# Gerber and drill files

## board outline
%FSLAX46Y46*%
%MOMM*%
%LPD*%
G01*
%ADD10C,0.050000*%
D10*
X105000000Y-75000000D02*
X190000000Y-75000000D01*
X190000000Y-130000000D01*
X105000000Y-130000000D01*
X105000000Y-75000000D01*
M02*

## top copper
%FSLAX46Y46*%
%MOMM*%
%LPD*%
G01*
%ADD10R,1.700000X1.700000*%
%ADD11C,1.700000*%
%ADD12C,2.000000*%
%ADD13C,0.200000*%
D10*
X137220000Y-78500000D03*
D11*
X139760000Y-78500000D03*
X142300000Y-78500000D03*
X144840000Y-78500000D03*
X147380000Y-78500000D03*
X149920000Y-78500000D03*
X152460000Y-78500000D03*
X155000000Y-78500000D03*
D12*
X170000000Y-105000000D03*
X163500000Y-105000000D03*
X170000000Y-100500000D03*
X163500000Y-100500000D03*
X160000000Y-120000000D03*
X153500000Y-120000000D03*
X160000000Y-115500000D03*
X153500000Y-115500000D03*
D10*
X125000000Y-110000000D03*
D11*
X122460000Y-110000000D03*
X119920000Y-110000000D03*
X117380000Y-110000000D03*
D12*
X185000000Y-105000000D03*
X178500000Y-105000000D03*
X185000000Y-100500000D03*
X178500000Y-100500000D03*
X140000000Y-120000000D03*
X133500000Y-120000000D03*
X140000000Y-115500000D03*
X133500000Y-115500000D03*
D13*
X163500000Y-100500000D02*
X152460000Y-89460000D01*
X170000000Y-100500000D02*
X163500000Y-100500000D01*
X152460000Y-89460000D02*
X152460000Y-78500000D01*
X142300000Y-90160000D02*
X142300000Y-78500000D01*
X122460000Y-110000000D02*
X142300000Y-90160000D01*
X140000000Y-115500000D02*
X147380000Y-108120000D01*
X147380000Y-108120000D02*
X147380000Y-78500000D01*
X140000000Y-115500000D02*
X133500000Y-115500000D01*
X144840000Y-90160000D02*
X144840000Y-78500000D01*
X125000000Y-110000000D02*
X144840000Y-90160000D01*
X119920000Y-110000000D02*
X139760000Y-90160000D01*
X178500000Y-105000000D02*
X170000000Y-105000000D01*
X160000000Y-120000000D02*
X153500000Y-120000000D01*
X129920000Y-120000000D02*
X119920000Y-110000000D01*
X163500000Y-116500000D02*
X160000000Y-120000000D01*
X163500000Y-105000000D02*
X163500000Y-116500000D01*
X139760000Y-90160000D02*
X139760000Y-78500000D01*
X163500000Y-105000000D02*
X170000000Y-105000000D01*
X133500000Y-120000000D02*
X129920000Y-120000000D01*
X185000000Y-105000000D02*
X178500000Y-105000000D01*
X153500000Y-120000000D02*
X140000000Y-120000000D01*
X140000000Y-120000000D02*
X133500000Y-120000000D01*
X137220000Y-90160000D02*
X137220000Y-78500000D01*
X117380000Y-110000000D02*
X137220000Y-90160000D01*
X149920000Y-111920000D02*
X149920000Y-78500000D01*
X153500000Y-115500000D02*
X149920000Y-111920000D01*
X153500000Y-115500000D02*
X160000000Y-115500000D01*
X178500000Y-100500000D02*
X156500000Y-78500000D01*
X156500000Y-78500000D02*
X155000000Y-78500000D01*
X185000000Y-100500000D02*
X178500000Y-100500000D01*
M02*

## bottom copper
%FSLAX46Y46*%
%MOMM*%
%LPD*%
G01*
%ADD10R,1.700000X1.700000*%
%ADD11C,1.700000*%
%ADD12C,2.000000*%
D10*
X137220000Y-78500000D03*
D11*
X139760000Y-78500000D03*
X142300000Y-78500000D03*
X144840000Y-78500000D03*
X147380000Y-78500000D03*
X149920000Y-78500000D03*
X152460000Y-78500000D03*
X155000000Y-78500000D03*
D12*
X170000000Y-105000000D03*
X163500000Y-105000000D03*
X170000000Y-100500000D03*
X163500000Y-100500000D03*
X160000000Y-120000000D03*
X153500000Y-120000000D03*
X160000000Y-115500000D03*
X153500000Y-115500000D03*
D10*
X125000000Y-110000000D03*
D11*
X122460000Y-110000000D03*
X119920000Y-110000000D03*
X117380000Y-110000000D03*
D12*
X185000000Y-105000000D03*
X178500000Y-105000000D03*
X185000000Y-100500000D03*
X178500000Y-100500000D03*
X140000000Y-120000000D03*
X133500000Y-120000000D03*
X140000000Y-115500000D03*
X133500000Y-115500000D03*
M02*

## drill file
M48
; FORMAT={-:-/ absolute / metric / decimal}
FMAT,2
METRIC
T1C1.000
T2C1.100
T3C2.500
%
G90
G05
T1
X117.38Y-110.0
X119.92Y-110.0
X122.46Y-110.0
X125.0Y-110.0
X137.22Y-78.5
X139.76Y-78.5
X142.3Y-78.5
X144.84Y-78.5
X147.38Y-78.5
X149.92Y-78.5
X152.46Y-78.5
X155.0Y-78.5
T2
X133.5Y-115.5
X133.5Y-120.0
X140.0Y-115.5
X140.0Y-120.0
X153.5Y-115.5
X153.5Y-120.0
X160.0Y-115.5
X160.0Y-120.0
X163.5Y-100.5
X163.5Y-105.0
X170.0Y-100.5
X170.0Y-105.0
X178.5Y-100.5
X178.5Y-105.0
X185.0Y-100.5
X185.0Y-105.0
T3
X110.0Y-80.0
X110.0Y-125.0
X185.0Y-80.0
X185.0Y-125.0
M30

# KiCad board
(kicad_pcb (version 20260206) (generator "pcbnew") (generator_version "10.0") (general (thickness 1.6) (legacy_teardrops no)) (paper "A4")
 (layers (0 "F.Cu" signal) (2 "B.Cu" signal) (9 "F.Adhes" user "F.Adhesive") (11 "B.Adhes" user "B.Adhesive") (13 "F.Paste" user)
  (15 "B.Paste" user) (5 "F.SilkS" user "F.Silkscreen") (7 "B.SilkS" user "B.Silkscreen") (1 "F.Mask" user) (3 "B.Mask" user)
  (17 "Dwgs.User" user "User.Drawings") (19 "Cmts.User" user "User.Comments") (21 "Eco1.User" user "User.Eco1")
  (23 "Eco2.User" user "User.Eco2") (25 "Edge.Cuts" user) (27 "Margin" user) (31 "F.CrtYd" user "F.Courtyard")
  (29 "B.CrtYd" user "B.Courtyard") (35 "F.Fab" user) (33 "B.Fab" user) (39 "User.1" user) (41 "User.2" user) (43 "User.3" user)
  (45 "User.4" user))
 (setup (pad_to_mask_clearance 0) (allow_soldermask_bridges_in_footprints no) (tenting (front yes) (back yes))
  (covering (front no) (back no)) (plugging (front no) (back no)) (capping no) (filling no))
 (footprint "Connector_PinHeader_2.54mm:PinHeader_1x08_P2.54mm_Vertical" (layer "F.Cu") (at 137.22 78.5 90)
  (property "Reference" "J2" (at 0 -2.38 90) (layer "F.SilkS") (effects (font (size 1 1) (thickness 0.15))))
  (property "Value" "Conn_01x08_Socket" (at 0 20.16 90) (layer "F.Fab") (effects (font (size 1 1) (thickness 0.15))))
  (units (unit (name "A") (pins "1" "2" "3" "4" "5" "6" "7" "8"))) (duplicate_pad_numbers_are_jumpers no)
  (pad "1" thru_hole rect (at 0 0 90) (size 1.7 1.7) (drill 1) (layers "*.Cu" "*.Mask") (remove_unused_layers no) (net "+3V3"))
  (pad "2" thru_hole circle (at 0 2.54 90) (size 1.7 1.7) (drill 1) (layers "*.Cu" "*.Mask") (remove_unused_layers no) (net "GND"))
  (pad "3" thru_hole circle (at 0 5.08 90) (size 1.7 1.7) (drill 1) (layers "*.Cu" "*.Mask") (remove_unused_layers no) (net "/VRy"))
  (pad "4" thru_hole circle (at 0 7.62 90) (size 1.7 1.7) (drill 1) (layers "*.Cu" "*.Mask") (remove_unused_layers no) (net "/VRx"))
  (pad "5" thru_hole circle (at 0 10.16 90) (size 1.7 1.7) (drill 1) (layers "*.Cu" "*.Mask") (remove_unused_layers no) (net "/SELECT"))
  (pad "6" thru_hole circle (at 0 12.7 90) (size 1.7 1.7) (drill 1) (layers "*.Cu" "*.Mask") (remove_unused_layers no) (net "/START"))
  (pad "7" thru_hole circle (at 0 15.24 90) (size 1.7 1.7) (drill 1) (layers "*.Cu" "*.Mask") (remove_unused_layers no) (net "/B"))
  (pad "8" thru_hole circle (at 0 17.78 90) (size 1.7 1.7) (drill 1) (layers "*.Cu" "*.Mask") (remove_unused_layers no) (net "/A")))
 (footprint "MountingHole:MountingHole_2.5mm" (layer "F.Cu") (at 185 125)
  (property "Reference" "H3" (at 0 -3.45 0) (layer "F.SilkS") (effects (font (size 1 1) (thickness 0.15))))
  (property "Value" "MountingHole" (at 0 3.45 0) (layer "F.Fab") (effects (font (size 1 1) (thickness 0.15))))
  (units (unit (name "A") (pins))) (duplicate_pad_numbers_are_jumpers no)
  (pad "" np_thru_hole circle (at 0 0) (size 2.5 2.5) (drill 2.5) (layers "*.Cu" "*.Mask")))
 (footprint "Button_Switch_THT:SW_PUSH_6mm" (layer "F.Cu") (at 170 105 180)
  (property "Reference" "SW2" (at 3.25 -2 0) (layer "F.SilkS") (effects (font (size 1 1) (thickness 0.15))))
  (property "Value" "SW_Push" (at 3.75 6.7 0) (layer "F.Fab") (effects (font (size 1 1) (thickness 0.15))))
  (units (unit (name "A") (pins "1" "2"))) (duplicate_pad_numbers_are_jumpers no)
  (pad "1" thru_hole circle (at 0 0 270) (size 2 2) (drill 1.1) (layers "*.Cu" "*.Mask") (remove_unused_layers no) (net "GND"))
  (pad "1" thru_hole circle (at 6.5 0 270) (size 2 2) (drill 1.1) (layers "*.Cu" "*.Mask") (remove_unused_layers no) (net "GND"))
  (pad "2" thru_hole circle (at 0 4.5 270) (size 2 2) (drill 1.1) (layers "*.Cu" "*.Mask") (remove_unused_layers no) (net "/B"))
  (pad "2" thru_hole circle (at 6.5 4.5 270) (size 2 2) (drill 1.1) (layers "*.Cu" "*.Mask") (remove_unused_layers no) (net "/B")))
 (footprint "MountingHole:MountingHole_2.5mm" (layer "F.Cu") (at 185 80)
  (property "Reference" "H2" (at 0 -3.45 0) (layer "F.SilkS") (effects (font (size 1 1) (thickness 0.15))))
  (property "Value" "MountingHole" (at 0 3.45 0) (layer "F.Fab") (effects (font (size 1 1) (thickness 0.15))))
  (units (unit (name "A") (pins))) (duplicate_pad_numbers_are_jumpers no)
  (pad "" np_thru_hole circle (at 0 0) (size 2.5 2.5) (drill 2.5) (layers "*.Cu" "*.Mask")))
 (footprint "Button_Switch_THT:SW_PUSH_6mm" (layer "F.Cu") (at 160 120 180)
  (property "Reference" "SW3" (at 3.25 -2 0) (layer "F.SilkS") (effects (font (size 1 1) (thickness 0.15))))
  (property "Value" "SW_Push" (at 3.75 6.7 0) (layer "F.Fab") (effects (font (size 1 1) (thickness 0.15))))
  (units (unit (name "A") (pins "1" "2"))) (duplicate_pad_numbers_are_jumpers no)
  (pad "1" thru_hole circle (at 0 0 270) (size 2 2) (drill 1.1) (layers "*.Cu" "*.Mask") (remove_unused_layers no) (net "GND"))
  (pad "1" thru_hole circle (at 6.5 0 270) (size 2 2) (drill 1.1) (layers "*.Cu" "*.Mask") (remove_unused_layers no) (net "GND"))
  (pad "2" thru_hole circle (at 0 4.5 270) (size 2 2) (drill 1.1) (layers "*.Cu" "*.Mask") (remove_unused_layers no) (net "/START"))
  (pad "2" thru_hole circle (at 6.5 4.5 270) (size 2 2) (drill 1.1) (layers "*.Cu" "*.Mask") (remove_unused_layers no) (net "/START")))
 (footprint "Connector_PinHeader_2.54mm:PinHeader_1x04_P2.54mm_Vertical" (layer "F.Cu") (at 125 110 -90)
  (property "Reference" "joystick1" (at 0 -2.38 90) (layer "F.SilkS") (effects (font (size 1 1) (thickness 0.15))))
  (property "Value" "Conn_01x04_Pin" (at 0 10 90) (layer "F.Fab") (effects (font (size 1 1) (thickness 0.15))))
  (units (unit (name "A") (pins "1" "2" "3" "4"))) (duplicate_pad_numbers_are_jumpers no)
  (pad "1" thru_hole rect (at 0 0 270) (size 1.7 1.7) (drill 1) (layers "*.Cu" "*.Mask") (remove_unused_layers no) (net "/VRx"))
  (pad "2" thru_hole circle (at 0 2.54 270) (size 1.7 1.7) (drill 1) (layers "*.Cu" "*.Mask") (remove_unused_layers no) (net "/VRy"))
  (pad "3" thru_hole circle (at 0 5.08 270) (size 1.7 1.7) (drill 1) (layers "*.Cu" "*.Mask") (remove_unused_layers no) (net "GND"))
  (pad "4" thru_hole circle (at 0 7.62 270) (size 1.7 1.7) (drill 1) (layers "*.Cu" "*.Mask") (remove_unused_layers no) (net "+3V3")))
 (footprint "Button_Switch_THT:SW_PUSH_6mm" (layer "F.Cu") (at 185 105 180)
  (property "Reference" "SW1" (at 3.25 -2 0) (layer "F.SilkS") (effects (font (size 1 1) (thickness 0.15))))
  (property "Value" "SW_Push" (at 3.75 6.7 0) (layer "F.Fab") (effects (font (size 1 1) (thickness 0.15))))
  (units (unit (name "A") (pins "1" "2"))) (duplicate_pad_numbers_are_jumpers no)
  (pad "1" thru_hole circle (at 0 0 270) (size 2 2) (drill 1.1) (layers "*.Cu" "*.Mask") (remove_unused_layers no) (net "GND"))
  (pad "1" thru_hole circle (at 6.5 0 270) (size 2 2) (drill 1.1) (layers "*.Cu" "*.Mask") (remove_unused_layers no) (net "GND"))
  (pad "2" thru_hole circle (at 0 4.5 270) (size 2 2) (drill 1.1) (layers "*.Cu" "*.Mask") (remove_unused_layers no) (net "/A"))
  (pad "2" thru_hole circle (at 6.5 4.5 270) (size 2 2) (drill 1.1) (layers "*.Cu" "*.Mask") (remove_unused_layers no) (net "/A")))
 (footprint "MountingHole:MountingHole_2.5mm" (layer "F.Cu") (at 110 80)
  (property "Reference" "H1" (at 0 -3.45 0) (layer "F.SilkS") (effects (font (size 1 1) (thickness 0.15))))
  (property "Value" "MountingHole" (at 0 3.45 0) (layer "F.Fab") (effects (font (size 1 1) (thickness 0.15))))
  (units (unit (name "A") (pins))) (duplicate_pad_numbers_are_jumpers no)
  (pad "" np_thru_hole circle (at 0 0) (size 2.5 2.5) (drill 2.5) (layers "*.Cu" "*.Mask")))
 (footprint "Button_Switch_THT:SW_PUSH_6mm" (layer "F.Cu") (at 140 120 180)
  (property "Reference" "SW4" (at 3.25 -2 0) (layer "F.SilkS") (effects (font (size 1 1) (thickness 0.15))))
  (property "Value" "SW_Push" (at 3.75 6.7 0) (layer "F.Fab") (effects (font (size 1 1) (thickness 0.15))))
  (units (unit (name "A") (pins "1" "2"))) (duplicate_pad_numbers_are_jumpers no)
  (pad "1" thru_hole circle (at 0 0 270) (size 2 2) (drill 1.1) (layers "*.Cu" "*.Mask") (remove_unused_layers no) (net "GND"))
  (pad "1" thru_hole circle (at 6.5 0 270) (size 2 2) (drill 1.1) (layers "*.Cu" "*.Mask") (remove_unused_layers no) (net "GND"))
  (pad "2" thru_hole circle (at 0 4.5 270) (size 2 2) (drill 1.1) (layers "*.Cu" "*.Mask") (remove_unused_layers no) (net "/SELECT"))
  (pad "2" thru_hole circle (at 6.5 4.5 270) (size 2 2) (drill 1.1) (layers "*.Cu" "*.Mask") (remove_unused_layers no) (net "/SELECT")))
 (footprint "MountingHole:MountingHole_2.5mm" (layer "F.Cu") (at 110 125)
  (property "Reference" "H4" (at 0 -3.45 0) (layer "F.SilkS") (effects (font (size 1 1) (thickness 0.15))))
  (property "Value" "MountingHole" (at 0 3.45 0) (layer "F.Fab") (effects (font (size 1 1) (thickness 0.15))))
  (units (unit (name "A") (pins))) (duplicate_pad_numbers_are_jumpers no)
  (pad "" np_thru_hole circle (at 0 0) (size 2.5 2.5) (drill 2.5) (layers "*.Cu" "*.Mask")))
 (gr_rect (start 105 75) (end 190 130) (stroke (width 0.05) (type default)) (fill no) (layer "Edge.Cuts"))
 (segment (start 163.5 100.5) (end 152.46 89.46) (width 0.2) (layer "F.Cu") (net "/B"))
 (segment (start 170 100.5) (end 163.5 100.5) (width 0.2) (layer "F.Cu") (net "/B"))
 (segment (start 152.46 89.46) (end 152.46 78.5) (width 0.2) (layer "F.Cu") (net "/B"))
 (segment (start 142.3 90.16) (end 142.3 78.5) (width 0.2) (layer "F.Cu") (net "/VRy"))
 (segment (start 122.46 110) (end 142.3 90.16) (width 0.2) (layer "F.Cu") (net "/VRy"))
 (segment (start 140 115.5) (end 147.38 108.12) (width 0.2) (layer "F.Cu") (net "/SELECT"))
 (segment (start 147.38 108.12) (end 147.38 78.5) (width 0.2) (layer "F.Cu") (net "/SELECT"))
 (segment (start 140 115.5) (end 133.5 115.5) (width 0.2) (layer "F.Cu") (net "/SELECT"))
 (segment (start 144.84 90.16) (end 144.84 78.5) (width 0.2) (layer "F.Cu") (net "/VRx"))
 (segment (start 125 110) (end 144.84 90.16) (width 0.2) (layer "F.Cu") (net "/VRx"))
 (segment (start 119.92 110) (end 139.76 90.16) (width 0.2) (layer "F.Cu") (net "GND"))
 (segment (start 178.5 105) (end 170 105) (width 0.2) (layer "F.Cu") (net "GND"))
 (segment (start 160 120) (end 153.5 120) (width 0.2) (layer "F.Cu") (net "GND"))
 (segment (start 129.92 120) (end 119.92 110) (width 0.2) (layer "F.Cu") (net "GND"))
 (segment (start 163.5 116.5) (end 160 120) (width 0.2) (layer "F.Cu") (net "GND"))
 (segment (start 163.5 105) (end 163.5 116.5) (width 0.2) (layer "F.Cu") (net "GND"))
 (segment (start 139.76 90.16) (end 139.76 78.5) (width 0.2) (layer "F.Cu") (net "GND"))
 (segment (start 163.5 105) (end 170 105) (width 0.2) (layer "F.Cu") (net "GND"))
 (segment (start 133.5 120) (end 129.92 120) (width 0.2) (layer "F.Cu") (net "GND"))
 (segment (start 185 105) (end 178.5 105) (width 0.2) (layer "F.Cu") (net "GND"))
 (segment (start 153.5 120) (end 140 120) (width 0.2) (layer "F.Cu") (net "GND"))
 (segment (start 140 120) (end 133.5 120) (width 0.2) (layer "F.Cu") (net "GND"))
 (segment (start 137.22 90.16) (end 137.22 78.5) (width 0.2) (layer "F.Cu") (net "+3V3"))
 (segment (start 117.38 110) (end 137.22 90.16) (width 0.2) (layer "F.Cu") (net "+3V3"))
 (segment (start 149.92 111.92) (end 149.92 78.5) (width 0.2) (layer "F.Cu") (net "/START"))
 (segment (start 153.5 115.5) (end 149.92 111.92) (width 0.2) (layer "F.Cu") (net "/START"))
 (segment (start 153.5 115.5) (end 160 115.5) (width 0.2) (layer "F.Cu") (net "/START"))
 (segment (start 178.5 100.5) (end 156.5 78.5) (width 0.2) (layer "F.Cu") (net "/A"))
 (segment (start 156.5 78.5) (end 155 78.5) (width 0.2) (layer "F.Cu") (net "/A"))
 (segment (start 185 100.5) (end 178.5 100.5) (width 0.2) (layer "F.Cu") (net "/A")))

